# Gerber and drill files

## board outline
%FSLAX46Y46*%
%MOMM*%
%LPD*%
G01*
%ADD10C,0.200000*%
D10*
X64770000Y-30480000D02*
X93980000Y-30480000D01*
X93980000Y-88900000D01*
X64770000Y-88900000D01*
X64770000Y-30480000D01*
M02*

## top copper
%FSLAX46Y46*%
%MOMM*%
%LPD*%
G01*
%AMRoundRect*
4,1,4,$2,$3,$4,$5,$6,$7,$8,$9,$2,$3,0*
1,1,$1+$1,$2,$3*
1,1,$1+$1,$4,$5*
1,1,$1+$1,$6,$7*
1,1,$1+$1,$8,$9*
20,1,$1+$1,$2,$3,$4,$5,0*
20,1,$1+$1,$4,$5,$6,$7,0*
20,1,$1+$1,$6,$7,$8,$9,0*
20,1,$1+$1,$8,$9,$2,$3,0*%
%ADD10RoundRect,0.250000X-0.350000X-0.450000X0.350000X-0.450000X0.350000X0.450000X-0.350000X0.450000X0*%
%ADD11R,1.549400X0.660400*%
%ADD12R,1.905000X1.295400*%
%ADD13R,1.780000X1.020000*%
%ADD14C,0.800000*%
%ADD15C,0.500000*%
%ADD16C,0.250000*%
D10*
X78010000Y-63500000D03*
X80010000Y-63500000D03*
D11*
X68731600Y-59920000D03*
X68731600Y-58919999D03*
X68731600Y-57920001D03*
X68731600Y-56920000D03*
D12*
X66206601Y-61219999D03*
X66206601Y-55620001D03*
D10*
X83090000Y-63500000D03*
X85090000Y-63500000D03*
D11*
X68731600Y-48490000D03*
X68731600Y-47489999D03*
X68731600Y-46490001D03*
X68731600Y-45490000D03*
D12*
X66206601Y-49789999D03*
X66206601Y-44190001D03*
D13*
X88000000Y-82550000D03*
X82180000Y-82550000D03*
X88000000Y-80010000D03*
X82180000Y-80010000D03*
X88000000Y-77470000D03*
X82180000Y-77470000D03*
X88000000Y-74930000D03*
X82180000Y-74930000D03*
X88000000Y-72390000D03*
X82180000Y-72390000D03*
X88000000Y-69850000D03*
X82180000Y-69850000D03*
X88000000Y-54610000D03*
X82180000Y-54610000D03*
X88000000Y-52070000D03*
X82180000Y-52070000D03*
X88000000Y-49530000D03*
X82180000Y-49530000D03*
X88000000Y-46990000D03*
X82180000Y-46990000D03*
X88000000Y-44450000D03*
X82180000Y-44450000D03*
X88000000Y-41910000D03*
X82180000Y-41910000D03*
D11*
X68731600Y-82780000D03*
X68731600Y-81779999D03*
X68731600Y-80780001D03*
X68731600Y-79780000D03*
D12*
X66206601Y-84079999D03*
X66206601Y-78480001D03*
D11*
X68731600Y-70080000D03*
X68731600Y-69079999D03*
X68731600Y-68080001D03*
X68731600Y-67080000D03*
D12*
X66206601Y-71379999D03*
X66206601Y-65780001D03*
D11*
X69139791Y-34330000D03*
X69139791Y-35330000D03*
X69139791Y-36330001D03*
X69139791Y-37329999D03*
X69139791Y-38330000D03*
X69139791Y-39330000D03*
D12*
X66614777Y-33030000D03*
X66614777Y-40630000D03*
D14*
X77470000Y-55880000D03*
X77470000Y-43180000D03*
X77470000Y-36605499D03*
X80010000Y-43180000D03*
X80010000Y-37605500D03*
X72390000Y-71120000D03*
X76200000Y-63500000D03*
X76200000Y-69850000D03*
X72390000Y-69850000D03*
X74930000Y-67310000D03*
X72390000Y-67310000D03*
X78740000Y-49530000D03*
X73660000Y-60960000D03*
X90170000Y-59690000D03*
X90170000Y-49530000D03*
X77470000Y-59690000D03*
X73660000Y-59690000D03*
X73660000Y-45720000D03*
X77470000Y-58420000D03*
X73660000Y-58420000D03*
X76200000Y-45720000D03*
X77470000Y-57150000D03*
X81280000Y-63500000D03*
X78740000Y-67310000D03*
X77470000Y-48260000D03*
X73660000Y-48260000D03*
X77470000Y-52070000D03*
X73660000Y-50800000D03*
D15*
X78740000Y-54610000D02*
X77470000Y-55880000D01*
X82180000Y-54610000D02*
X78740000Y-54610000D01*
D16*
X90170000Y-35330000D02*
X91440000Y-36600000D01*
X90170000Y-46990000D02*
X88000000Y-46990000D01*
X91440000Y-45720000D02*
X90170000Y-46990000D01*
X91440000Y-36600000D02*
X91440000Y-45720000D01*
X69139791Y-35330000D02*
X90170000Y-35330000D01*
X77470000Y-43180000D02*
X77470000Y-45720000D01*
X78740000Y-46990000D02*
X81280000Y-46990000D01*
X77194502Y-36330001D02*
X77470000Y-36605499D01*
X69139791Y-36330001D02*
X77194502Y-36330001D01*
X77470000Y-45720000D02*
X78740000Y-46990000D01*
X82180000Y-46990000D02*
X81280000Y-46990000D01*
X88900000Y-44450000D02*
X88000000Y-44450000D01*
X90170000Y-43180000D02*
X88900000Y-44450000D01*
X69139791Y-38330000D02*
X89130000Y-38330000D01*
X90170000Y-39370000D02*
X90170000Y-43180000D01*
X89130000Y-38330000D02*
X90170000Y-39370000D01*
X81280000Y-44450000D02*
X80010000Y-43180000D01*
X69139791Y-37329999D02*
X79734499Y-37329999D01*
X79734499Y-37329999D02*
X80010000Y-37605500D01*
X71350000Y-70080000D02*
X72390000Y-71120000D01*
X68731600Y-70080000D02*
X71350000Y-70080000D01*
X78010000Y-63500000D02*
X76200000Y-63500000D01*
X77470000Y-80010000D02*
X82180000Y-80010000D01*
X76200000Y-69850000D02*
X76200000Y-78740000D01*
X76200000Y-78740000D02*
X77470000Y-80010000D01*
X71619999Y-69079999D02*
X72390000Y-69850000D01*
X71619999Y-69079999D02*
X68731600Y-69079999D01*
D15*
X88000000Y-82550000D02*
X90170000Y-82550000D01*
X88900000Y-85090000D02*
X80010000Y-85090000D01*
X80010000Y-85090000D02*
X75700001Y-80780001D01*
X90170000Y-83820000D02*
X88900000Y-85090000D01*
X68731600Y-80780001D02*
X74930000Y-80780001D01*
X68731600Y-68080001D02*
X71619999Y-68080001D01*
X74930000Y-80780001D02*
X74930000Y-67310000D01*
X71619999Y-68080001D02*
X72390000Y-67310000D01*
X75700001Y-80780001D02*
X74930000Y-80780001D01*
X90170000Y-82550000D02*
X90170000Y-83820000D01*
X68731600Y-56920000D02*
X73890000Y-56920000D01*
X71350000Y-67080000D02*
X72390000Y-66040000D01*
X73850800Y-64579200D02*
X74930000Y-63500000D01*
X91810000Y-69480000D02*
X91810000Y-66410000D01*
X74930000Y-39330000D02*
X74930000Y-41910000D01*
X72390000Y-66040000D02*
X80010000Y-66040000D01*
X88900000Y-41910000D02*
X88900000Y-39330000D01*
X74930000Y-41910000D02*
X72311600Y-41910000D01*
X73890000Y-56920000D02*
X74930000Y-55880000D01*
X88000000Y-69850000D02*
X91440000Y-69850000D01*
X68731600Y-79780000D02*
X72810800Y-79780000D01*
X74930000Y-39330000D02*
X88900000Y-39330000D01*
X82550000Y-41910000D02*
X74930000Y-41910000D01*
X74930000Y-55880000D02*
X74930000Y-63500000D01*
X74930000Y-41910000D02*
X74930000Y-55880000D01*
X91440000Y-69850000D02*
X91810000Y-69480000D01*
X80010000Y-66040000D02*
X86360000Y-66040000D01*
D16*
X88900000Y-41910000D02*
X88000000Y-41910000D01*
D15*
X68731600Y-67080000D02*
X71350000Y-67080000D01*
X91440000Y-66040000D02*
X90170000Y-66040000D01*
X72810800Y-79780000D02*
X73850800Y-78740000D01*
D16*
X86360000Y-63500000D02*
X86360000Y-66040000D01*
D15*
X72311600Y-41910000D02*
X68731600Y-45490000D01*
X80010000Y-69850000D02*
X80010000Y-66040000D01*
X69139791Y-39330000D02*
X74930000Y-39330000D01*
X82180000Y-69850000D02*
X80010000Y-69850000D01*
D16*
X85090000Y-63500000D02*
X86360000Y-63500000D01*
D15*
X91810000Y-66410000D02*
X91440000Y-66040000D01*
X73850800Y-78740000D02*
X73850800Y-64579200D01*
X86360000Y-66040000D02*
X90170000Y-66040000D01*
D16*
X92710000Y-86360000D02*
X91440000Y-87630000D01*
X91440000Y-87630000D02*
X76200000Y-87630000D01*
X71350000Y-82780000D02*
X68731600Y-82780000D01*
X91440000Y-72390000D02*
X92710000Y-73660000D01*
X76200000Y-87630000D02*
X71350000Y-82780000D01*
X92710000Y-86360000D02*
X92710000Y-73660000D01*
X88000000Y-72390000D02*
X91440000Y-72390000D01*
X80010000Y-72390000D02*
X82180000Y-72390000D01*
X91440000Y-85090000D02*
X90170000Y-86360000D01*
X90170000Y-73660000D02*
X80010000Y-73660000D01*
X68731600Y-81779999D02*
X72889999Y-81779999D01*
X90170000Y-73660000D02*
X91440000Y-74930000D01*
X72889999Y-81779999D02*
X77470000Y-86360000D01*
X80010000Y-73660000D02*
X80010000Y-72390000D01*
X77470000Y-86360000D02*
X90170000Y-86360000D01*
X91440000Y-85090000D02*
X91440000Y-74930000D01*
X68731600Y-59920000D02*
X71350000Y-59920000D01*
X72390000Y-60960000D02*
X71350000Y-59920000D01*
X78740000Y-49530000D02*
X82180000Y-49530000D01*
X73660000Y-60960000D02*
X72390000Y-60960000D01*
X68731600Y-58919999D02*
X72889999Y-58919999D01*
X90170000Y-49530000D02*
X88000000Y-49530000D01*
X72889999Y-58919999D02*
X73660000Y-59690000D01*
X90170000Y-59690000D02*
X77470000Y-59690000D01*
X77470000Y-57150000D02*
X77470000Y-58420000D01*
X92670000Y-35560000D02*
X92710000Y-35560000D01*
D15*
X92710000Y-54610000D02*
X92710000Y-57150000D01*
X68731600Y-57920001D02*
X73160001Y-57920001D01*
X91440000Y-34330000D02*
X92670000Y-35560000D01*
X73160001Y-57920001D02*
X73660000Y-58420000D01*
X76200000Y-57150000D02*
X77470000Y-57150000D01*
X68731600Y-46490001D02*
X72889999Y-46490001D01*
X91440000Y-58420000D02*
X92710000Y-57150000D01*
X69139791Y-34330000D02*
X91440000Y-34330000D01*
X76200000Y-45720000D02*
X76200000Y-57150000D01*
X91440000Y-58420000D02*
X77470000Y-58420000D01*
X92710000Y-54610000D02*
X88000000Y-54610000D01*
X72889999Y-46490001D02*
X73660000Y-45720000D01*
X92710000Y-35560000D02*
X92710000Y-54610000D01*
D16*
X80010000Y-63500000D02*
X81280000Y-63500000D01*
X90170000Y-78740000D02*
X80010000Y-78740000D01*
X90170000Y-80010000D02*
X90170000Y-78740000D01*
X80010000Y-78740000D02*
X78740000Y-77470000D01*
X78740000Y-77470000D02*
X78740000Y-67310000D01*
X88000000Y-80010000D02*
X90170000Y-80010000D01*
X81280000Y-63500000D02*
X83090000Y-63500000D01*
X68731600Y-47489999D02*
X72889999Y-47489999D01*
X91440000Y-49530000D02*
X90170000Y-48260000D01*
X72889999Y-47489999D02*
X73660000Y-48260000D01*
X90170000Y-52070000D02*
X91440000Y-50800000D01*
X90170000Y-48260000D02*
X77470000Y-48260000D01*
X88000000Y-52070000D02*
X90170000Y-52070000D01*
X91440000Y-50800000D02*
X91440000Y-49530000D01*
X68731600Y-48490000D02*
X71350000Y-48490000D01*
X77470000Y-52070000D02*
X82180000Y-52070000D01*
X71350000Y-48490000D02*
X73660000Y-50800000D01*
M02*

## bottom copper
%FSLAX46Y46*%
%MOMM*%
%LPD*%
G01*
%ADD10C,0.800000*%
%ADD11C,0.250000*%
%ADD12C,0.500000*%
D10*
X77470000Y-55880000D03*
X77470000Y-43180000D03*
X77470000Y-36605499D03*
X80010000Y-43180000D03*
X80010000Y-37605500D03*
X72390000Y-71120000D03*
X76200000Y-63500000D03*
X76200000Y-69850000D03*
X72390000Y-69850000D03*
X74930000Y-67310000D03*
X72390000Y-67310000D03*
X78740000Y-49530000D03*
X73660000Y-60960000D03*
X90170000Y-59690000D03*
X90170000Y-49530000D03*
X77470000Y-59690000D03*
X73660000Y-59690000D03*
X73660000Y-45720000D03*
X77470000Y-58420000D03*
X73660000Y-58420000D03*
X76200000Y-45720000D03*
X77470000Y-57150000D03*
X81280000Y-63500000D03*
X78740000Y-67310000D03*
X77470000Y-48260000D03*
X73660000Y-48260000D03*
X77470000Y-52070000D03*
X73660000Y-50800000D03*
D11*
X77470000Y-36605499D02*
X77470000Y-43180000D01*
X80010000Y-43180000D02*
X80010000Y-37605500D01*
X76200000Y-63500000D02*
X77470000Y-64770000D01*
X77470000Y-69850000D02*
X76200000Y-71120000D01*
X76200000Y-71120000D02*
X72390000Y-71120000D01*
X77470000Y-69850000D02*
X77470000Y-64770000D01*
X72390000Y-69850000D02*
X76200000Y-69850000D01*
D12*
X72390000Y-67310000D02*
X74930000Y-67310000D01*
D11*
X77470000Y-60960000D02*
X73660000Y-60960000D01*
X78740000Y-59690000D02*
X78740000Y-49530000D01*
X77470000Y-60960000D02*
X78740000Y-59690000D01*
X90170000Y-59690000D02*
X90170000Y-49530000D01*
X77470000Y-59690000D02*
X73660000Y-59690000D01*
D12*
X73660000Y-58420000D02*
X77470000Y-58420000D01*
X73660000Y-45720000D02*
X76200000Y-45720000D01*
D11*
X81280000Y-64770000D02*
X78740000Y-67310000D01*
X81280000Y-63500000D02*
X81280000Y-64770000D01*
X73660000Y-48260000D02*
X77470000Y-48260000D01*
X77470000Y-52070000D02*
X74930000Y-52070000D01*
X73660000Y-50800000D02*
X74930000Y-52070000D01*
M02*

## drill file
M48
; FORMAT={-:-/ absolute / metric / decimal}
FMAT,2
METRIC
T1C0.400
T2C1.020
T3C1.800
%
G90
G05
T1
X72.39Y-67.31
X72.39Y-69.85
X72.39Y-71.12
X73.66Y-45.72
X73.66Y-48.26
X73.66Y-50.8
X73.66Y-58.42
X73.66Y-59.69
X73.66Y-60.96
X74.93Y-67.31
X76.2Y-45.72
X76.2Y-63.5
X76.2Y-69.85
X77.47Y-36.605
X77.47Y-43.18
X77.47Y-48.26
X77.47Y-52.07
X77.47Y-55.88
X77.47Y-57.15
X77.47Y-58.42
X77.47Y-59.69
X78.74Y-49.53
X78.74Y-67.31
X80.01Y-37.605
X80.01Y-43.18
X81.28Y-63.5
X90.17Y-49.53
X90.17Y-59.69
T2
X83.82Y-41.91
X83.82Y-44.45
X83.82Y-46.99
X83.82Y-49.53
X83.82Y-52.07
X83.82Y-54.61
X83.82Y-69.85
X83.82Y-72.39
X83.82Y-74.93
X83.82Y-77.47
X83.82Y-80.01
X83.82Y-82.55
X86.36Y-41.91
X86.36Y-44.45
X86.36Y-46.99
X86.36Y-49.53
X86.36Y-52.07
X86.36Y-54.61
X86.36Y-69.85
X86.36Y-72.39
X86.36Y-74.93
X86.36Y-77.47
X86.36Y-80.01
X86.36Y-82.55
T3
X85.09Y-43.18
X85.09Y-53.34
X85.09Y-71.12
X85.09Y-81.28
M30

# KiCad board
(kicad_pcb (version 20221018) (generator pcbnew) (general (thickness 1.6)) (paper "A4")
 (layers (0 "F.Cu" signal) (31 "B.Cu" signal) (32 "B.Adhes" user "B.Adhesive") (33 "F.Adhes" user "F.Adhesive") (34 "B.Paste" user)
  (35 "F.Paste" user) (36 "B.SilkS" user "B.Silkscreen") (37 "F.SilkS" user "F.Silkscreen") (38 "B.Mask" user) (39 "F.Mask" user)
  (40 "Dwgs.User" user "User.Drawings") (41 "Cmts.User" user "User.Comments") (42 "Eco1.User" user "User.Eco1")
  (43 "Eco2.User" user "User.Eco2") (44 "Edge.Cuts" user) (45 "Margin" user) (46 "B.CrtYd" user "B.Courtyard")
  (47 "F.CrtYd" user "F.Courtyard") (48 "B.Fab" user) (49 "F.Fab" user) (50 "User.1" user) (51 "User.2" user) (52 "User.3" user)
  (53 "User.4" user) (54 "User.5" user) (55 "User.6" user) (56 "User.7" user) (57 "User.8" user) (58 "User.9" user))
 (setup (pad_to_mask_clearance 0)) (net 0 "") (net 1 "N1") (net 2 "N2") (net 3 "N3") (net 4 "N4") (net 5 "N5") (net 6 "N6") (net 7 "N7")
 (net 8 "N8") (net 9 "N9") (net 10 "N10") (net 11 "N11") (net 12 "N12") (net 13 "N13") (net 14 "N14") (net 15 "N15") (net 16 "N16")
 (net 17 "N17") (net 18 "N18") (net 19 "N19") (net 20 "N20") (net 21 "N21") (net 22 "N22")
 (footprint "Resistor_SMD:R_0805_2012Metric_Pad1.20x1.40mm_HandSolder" (layer "F.Cu") (at 79.01 63.5)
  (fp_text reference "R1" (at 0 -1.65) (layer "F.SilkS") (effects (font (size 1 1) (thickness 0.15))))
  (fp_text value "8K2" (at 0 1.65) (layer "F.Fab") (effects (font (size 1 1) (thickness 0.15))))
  (pad "1" smd roundrect (at -1 0) (size 1.2 1.4) (layers "F.Cu" "F.Paste" "F.Mask") (roundrect_rratio 0.2083333333) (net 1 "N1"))
  (pad "2" smd roundrect (at 1 0) (size 1.2 1.4) (layers "F.Cu" "F.Paste" "F.Mask") (roundrect_rratio 0.2083333333) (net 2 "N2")))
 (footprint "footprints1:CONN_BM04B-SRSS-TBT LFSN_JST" (layer "F.Cu") (at 67.31 58.42 90)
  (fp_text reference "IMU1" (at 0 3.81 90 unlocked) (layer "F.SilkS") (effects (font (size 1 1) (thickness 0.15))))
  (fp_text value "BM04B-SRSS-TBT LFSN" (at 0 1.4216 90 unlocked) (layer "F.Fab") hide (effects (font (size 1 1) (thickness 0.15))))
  (pad "1" smd rect (at -1.5 1.4216 90) (size 0.6604 1.5494) (layers "F.Cu" "F.Paste" "F.Mask") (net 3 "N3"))
  (pad "2" smd rect (at -0.499999 1.4216 90) (size 0.6604 1.5494) (layers "F.Cu" "F.Paste" "F.Mask") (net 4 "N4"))
  (pad "3" smd rect (at 0.499999 1.4216 90) (size 0.6604 1.5494) (layers "F.Cu" "F.Paste" "F.Mask") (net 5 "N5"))
  (pad "4" smd rect (at 1.5 1.4216 90) (size 0.6604 1.5494) (layers "F.Cu" "F.Paste" "F.Mask") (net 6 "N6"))
  (pad "5" smd rect (at -2.799999 -1.103399 180) (size 1.905 1.2954) (layers "F.Cu" "F.Paste" "F.Mask"))
  (pad "6" smd rect (at 2.799999 -1.103399 180) (size 1.905 1.2954) (layers "F.Cu" "F.Paste" "F.Mask")))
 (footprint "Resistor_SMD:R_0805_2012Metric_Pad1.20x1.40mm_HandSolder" (layer "F.Cu") (at 84.09 63.5)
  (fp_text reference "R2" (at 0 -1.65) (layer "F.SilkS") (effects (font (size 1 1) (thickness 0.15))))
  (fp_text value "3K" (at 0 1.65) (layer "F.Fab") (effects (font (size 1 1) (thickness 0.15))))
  (pad "1" smd roundrect (at -1 0) (size 1.2 1.4) (layers "F.Cu" "F.Paste" "F.Mask") (roundrect_rratio 0.2083333333) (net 2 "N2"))
  (pad "2" smd roundrect (at 1 0) (size 1.2 1.4) (layers "F.Cu" "F.Paste" "F.Mask") (roundrect_rratio 0.2083333333) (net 6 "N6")))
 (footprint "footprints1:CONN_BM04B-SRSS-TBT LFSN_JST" (layer "F.Cu") (at 67.31 46.99 90)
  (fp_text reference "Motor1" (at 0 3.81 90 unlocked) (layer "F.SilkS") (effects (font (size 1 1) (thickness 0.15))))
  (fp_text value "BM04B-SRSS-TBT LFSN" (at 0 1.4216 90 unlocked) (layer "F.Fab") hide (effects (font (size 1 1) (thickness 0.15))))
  (pad "1" smd rect (at -1.5 1.4216 90) (size 0.6604 1.5494) (layers "F.Cu" "F.Paste" "F.Mask") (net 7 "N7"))
  (pad "2" smd rect (at -0.499999 1.4216 90) (size 0.6604 1.5494) (layers "F.Cu" "F.Paste" "F.Mask") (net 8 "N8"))
  (pad "3" smd rect (at 0.499999 1.4216 90) (size 0.6604 1.5494) (layers "F.Cu" "F.Paste" "F.Mask") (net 5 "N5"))
  (pad "4" smd rect (at 1.5 1.4216 90) (size 0.6604 1.5494) (layers "F.Cu" "F.Paste" "F.Mask") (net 6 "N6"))
  (pad "5" smd rect (at -2.799999 -1.103399 180) (size 1.905 1.2954) (layers "F.Cu" "F.Paste" "F.Mask"))
  (pad "6" smd rect (at 2.799999 -1.103399 180) (size 1.905 1.2954) (layers "F.Cu" "F.Paste" "F.Mask")))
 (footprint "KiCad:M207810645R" (layer "F.Cu") (at 85.09 76.2 90)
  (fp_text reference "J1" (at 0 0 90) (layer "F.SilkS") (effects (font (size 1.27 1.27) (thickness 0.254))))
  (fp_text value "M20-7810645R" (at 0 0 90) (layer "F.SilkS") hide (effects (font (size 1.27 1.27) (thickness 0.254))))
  (pad "" np_thru_hole circle (at -6.35 -1.27 90) (size 1.02 1.02) (drill 1.02) (layers "*.Cu" "*.Mask"))
  (pad "" np_thru_hole circle (at -6.35 1.27 90) (size 1.02 1.02) (drill 1.02) (layers "*.Cu" "*.Mask"))
  (pad "" np_thru_hole circle (at -5.08 0 90) (size 1.8 1.8) (drill 1.8) (layers "*.Cu" "*.Mask"))
  (pad "" np_thru_hole circle (at -3.81 -1.27 90) (size 1.02 1.02) (drill 1.02) (layers "*.Cu" "*.Mask"))
  (pad "" np_thru_hole circle (at -3.81 1.27 90) (size 1.02 1.02) (drill 1.02) (layers "*.Cu" "*.Mask"))
  (pad "" np_thru_hole circle (at -1.27 -1.27 90) (size 1.02 1.02) (drill 1.02) (layers "*.Cu" "*.Mask"))
  (pad "" np_thru_hole circle (at -1.27 1.27 90) (size 1.02 1.02) (drill 1.02) (layers "*.Cu" "*.Mask"))
  (pad "" np_thru_hole circle (at 1.27 -1.27 90) (size 1.02 1.02) (drill 1.02) (layers "*.Cu" "*.Mask"))
  (pad "" np_thru_hole circle (at 1.27 1.27 90) (size 1.02 1.02) (drill 1.02) (layers "*.Cu" "*.Mask"))
  (pad "" np_thru_hole circle (at 3.81 -1.27 90) (size 1.02 1.02) (drill 1.02) (layers "*.Cu" "*.Mask"))
  (pad "" np_thru_hole circle (at 3.81 1.27 90) (size 1.02 1.02) (drill 1.02) (layers "*.Cu" "*.Mask"))
  (pad "" np_thru_hole circle (at 5.08 0 90) (size 1.8 1.8) (drill 1.8) (layers "*.Cu" "*.Mask"))
  (pad "" np_thru_hole circle (at 6.35 -1.27 90) (size 1.02 1.02) (drill 1.02) (layers "*.Cu" "*.Mask"))
  (pad "" np_thru_hole circle (at 6.35 1.27 90) (size 1.02 1.02) (drill 1.02) (layers "*.Cu" "*.Mask"))
  (pad "1" smd rect (at -6.35 2.91 90) (size 1.02 1.78) (layers "F.Cu" "F.Paste" "F.Mask") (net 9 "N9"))
  (pad "2" smd rect (at -6.35 -2.91 90) (size 1.02 1.78) (layers "F.Cu" "F.Paste" "F.Mask") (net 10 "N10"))
  (pad "3" smd rect (at -3.81 2.91 90) (size 1.02 1.78) (layers "F.Cu" "F.Paste" "F.Mask") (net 2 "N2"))
  (pad "4" smd rect (at -3.81 -2.91 90) (size 1.02 1.78) (layers "F.Cu" "F.Paste" "F.Mask") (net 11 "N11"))
  (pad "5" smd rect (at -1.27 2.91 90) (size 1.02 1.78) (layers "F.Cu" "F.Paste" "F.Mask") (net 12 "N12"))
  (pad "6" smd rect (at -1.27 -2.91 90) (size 1.02 1.78) (layers "F.Cu" "F.Paste" "F.Mask") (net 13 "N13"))
  (pad "7" smd rect (at 1.27 2.91 90) (size 1.02 1.78) (layers "F.Cu" "F.Paste" "F.Mask") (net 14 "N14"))
  (pad "8" smd rect (at 1.27 -2.91 90) (size 1.02 1.78) (layers "F.Cu" "F.Paste" "F.Mask") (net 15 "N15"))
  (pad "9" smd rect (at 3.81 2.91 90) (size 1.02 1.78) (layers "F.Cu" "F.Paste" "F.Mask") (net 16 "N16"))
  (pad "10" smd rect (at 3.81 -2.91 90) (size 1.02 1.78) (layers "F.Cu" "F.Paste" "F.Mask") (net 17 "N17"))
  (pad "11" smd rect (at 6.35 2.91 90) (size 1.02 1.78) (layers "F.Cu" "F.Paste" "F.Mask") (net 6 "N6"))
  (pad "12" smd rect (at 6.35 -2.91 90) (size 1.02 1.78) (layers "F.Cu" "F.Paste" "F.Mask") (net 6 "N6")))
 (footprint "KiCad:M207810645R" (layer "F.Cu") (at 85.09 48.26 90)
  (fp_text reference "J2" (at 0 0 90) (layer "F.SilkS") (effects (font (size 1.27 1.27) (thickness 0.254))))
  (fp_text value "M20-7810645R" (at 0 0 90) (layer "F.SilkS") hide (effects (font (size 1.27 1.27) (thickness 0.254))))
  (pad "" np_thru_hole circle (at -6.35 -1.27 90) (size 1.02 1.02) (drill 1.02) (layers "*.Cu" "*.Mask"))
  (pad "" np_thru_hole circle (at -6.35 1.27 90) (size 1.02 1.02) (drill 1.02) (layers "*.Cu" "*.Mask"))
  (pad "" np_thru_hole circle (at -5.08 0 90) (size 1.8 1.8) (drill 1.8) (layers "*.Cu" "*.Mask"))
  (pad "" np_thru_hole circle (at -3.81 -1.27 90) (size 1.02 1.02) (drill 1.02) (layers "*.Cu" "*.Mask"))
  (pad "" np_thru_hole circle (at -3.81 1.27 90) (size 1.02 1.02) (drill 1.02) (layers "*.Cu" "*.Mask"))
  (pad "" np_thru_hole circle (at -1.27 -1.27 90) (size 1.02 1.02) (drill 1.02) (layers "*.Cu" "*.Mask"))
  (pad "" np_thru_hole circle (at -1.27 1.27 90) (size 1.02 1.02) (drill 1.02) (layers "*.Cu" "*.Mask"))
  (pad "" np_thru_hole circle (at 1.27 -1.27 90) (size 1.02 1.02) (drill 1.02) (layers "*.Cu" "*.Mask"))
  (pad "" np_thru_hole circle (at 1.27 1.27 90) (size 1.02 1.02) (drill 1.02) (layers "*.Cu" "*.Mask"))
  (pad "" np_thru_hole circle (at 3.81 -1.27 90) (size 1.02 1.02) (drill 1.02) (layers "*.Cu" "*.Mask"))
  (pad "" np_thru_hole circle (at 3.81 1.27 90) (size 1.02 1.02) (drill 1.02) (layers "*.Cu" "*.Mask"))
  (pad "" np_thru_hole circle (at 5.08 0 90) (size 1.8 1.8) (drill 1.8) (layers "*.Cu" "*.Mask"))
  (pad "" np_thru_hole circle (at 6.35 -1.27 90) (size 1.02 1.02) (drill 1.02) (layers "*.Cu" "*.Mask"))
  (pad "" np_thru_hole circle (at 6.35 1.27 90) (size 1.02 1.02) (drill 1.02) (layers "*.Cu" "*.Mask"))
  (pad "1" smd rect (at -6.35 2.91 90) (size 1.02 1.78) (layers "F.Cu" "F.Paste" "F.Mask") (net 5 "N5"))
  (pad "2" smd rect (at -6.35 -2.91 90) (size 1.02 1.78) (layers "F.Cu" "F.Paste" "F.Mask") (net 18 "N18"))
  (pad "3" smd rect (at -3.81 2.91 90) (size 1.02 1.78) (layers "F.Cu" "F.Paste" "F.Mask") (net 8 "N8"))
  (pad "4" smd rect (at -3.81 -2.91 90) (size 1.02 1.78) (layers "F.Cu" "F.Paste" "F.Mask") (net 7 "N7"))
  (pad "5" smd rect (at -1.27 2.91 90) (size 1.02 1.78) (layers "F.Cu" "F.Paste" "F.Mask") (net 4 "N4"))
  (pad "6" smd rect (at -1.27 -2.91 90) (size 1.02 1.78) (layers "F.Cu" "F.Paste" "F.Mask") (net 3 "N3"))
  (pad "7" smd rect (at 1.27 2.91 90) (size 1.02 1.78) (layers "F.Cu" "F.Paste" "F.Mask") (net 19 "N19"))
  (pad "8" smd rect (at 1.27 -2.91 90) (size 1.02 1.78) (layers "F.Cu" "F.Paste" "F.Mask") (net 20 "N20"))
  (pad "9" smd rect (at 3.81 2.91 90) (size 1.02 1.78) (layers "F.Cu" "F.Paste" "F.Mask") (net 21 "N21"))
  (pad "10" smd rect (at 3.81 -2.91 90) (size 1.02 1.78) (layers "F.Cu" "F.Paste" "F.Mask") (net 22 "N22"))
  (pad "11" smd rect (at 6.35 2.91 90) (size 1.02 1.78) (layers "F.Cu" "F.Paste" "F.Mask") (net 6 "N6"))
  (pad "12" smd rect (at 6.35 -2.91 90) (size 1.02 1.78) (layers "F.Cu" "F.Paste" "F.Mask") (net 6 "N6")))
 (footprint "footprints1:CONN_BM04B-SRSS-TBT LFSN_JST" (layer "F.Cu") (at 67.31 81.28 90)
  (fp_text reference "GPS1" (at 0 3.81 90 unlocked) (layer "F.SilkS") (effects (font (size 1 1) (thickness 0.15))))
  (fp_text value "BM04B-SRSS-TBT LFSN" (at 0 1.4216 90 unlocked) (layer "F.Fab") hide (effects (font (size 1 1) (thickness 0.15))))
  (pad "1" smd rect (at -1.5 1.4216 90) (size 0.6604 1.5494) (layers "F.Cu" "F.Paste" "F.Mask") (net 16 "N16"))
  (pad "2" smd rect (at -0.499999 1.4216 90) (size 0.6604 1.5494) (layers "F.Cu" "F.Paste" "F.Mask") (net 17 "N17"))
  (pad "3" smd rect (at 0.499999 1.4216 90) (size 0.6604 1.5494) (layers "F.Cu" "F.Paste" "F.Mask") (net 9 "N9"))
  (pad "4" smd rect (at 1.5 1.4216 90) (size 0.6604 1.5494) (layers "F.Cu" "F.Paste" "F.Mask") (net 6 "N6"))
  (pad "5" smd rect (at -2.799999 -1.103399 180) (size 1.905 1.2954) (layers "F.Cu" "F.Paste" "F.Mask"))
  (pad "6" smd rect (at 2.799999 -1.103399 180) (size 1.905 1.2954) (layers "F.Cu" "F.Paste" "F.Mask")))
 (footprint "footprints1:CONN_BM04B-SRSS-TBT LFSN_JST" (layer "F.Cu") (at 67.31 68.58 90)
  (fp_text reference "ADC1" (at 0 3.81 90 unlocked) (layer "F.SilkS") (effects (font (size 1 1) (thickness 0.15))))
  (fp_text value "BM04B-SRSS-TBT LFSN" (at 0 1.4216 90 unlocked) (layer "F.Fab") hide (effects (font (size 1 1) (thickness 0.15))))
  (pad "1" smd rect (at -1.5 1.4216 90) (size 0.6604 1.5494) (layers "F.Cu" "F.Paste" "F.Mask") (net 1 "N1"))
  (pad "2" smd rect (at -0.499999 1.4216 90) (size 0.6604 1.5494) (layers "F.Cu" "F.Paste" "F.Mask") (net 11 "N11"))
  (pad "3" smd rect (at 0.499999 1.4216 90) (size 0.6604 1.5494) (layers "F.Cu" "F.Paste" "F.Mask") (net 9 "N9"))
  (pad "4" smd rect (at 1.5 1.4216 90) (size 0.6604 1.5494) (layers "F.Cu" "F.Paste" "F.Mask") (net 6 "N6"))
  (pad "5" smd rect (at -2.799999 -1.103399 180) (size 1.905 1.2954) (layers "F.Cu" "F.Paste" "F.Mask"))
  (pad "6" smd rect (at 2.799999 -1.103399 180) (size 1.905 1.2954) (layers "F.Cu" "F.Paste" "F.Mask")))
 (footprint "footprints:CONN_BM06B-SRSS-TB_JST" (layer "F.Cu") (at 67.31 36.83 -90)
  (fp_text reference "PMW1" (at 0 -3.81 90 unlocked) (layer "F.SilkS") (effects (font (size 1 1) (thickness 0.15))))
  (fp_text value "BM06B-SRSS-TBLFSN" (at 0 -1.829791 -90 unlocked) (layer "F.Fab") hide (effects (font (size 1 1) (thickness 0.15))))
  (pad "1" smd rect (at -2.5 -1.829791 270) (size 0.6604 1.5494) (layers "F.Cu" "F.Paste" "F.Mask") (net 5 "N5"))
  (pad "2" smd rect (at -1.5 -1.829791 270) (size 0.6604 1.5494) (layers "F.Cu" "F.Paste" "F.Mask") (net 19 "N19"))
  (pad "3" smd rect (at -0.499999 -1.829791 270) (size 0.6604 1.5494) (layers "F.Cu" "F.Paste" "F.Mask") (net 20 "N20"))
  (pad "4" smd rect (at 0.499999 -1.829791 270) (size 0.6604 1.5494) (layers "F.Cu" "F.Paste" "F.Mask") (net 22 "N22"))
  (pad "5" smd rect (at 1.5 -1.829791 270) (size 0.6604 1.5494) (layers "F.Cu" "F.Paste" "F.Mask") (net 21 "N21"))
  (pad "6" smd rect (at 2.5 -1.829791 270) (size 0.6604 1.5494) (layers "F.Cu" "F.Paste" "F.Mask") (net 6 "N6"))
  (pad "7" smd rect (at -3.8 0.695223) (size 1.905 1.2954) (layers "F.Cu" "F.Paste" "F.Mask"))
  (pad "8" smd rect (at 3.8 0.695223) (size 1.905 1.2954) (layers "F.Cu" "F.Paste" "F.Mask")))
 (gr_rect (start 64.77 30.48) (end 93.98 88.9) (stroke (width 0.2) (type default)) (fill none) (layer "Edge.Cuts"))
 (segment (start 78.74 54.61) (end 77.47 55.88) (width 0.5) (layer "F.Cu") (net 18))
 (segment (start 82.18 54.61) (end 78.74 54.61) (width 0.5) (layer "F.Cu") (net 18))
 (via (at 77.47 55.88) (size 0.8) (drill 0.4) (layers "F.Cu" "B.Cu") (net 18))
 (segment (start 90.17 35.33) (end 91.44 36.6) (width 0.25) (layer "F.Cu") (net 19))
 (segment (start 90.17 46.99) (end 88 46.99) (width 0.25) (layer "F.Cu") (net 19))
 (segment (start 91.44 45.72) (end 90.17 46.99) (width 0.25) (layer "F.Cu") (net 19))
 (segment (start 91.44 36.6) (end 91.44 45.72) (width 0.25) (layer "F.Cu") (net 19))
 (segment (start 69.139791 35.33) (end 90.17 35.33) (width 0.25) (layer "F.Cu") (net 19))
 (segment (start 77.47 43.18) (end 77.47 45.72) (width 0.25) (layer "F.Cu") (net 20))
 (segment (start 78.74 46.99) (end 81.28 46.99) (width 0.25) (layer "F.Cu") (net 20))
 (segment (start 77.194502 36.330001) (end 77.47 36.605499) (width 0.25) (layer "F.Cu") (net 20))
 (segment (start 69.139791 36.330001) (end 77.194502 36.330001) (width 0.25) (layer "F.Cu") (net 20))
 (segment (start 77.47 45.72) (end 78.74 46.99) (width 0.25) (layer "F.Cu") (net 20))
 (segment (start 82.18 46.99) (end 81.28 46.99) (width 0.25) (layer "F.Cu") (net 20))
 (via (at 77.47 43.18) (size 0.8) (drill 0.4) (layers "F.Cu" "B.Cu") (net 20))
 (via (at 77.47 36.605499) (size 0.8) (drill 0.4) (layers "F.Cu" "B.Cu") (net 20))
 (segment (start 77.47 36.605499) (end 77.47 43.18) (width 0.25) (layer "B.Cu") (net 20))
 (segment (start 88.9 44.45) (end 88 44.45) (width 0.25) (layer "F.Cu") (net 21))
 (segment (start 90.17 43.18) (end 88.9 44.45) (width 0.25) (layer "F.Cu") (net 21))
 (segment (start 69.139791 38.33) (end 89.13 38.33) (width 0.25) (layer "F.Cu") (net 21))
 (segment (start 90.17 39.37) (end 90.17 43.18) (width 0.25) (layer "F.Cu") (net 21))
 (segment (start 89.13 38.33) (end 90.17 39.37) (width 0.25) (layer "F.Cu") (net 21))
 (segment (start 81.28 44.45) (end 80.01 43.18) (width 0.25) (layer "F.Cu") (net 22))
 (segment (start 69.139791 37.329999) (end 79.734499 37.329999) (width 0.25) (layer "F.Cu") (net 22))
 (segment (start 79.734499 37.329999) (end 80.01 37.6055) (width 0.25) (layer "F.Cu") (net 22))
 (via (at 80.01 43.18) (size 0.8) (drill 0.4) (layers "F.Cu" "B.Cu") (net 22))
 (via (at 80.01 37.6055) (size 0.8) (drill 0.4) (layers "F.Cu" "B.Cu") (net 22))
 (segment (start 80.01 43.18) (end 80.01 37.6055) (width 0.25) (layer "B.Cu") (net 22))
 (segment (start 71.35 70.08) (end 72.39 71.12) (width 0.25) (layer "F.Cu") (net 1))
 (segment (start 68.7316 70.08) (end 71.35 70.08) (width 0.25) (layer "F.Cu") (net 1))
 (segment (start 78.01 63.5) (end 76.2 63.5) (width 0.25) (layer "F.Cu") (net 1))
 (via (at 72.39 71.12) (size 0.8) (drill 0.4) (layers "F.Cu" "B.Cu") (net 1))
 (via (at 76.2 63.5) (size 0.8) (drill 0.4) (layers "F.Cu" "B.Cu") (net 1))
 (segment (start 76.2 63.5) (end 77.47 64.77) (width 0.25) (layer "B.Cu") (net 1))
 (segment (start 77.47 69.85) (end 76.2 71.12) (width 0.25) (layer "B.Cu") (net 1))
 (segment (start 76.2 71.12) (end 72.39 71.12) (width 0.25) (layer "B.Cu") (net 1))
 (segment (start 77.47 69.85) (end 77.47 64.77) (width 0.25) (layer "B.Cu") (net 1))
 (segment (start 77.47 80.01) (end 82.18 80.01) (width 0.25) (layer "F.Cu") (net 11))
 (segment (start 76.2 69.85) (end 76.2 78.74) (width 0.25) (layer "F.Cu") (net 11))
 (segment (start 76.2 78.74) (end 77.47 80.01) (width 0.25) (layer "F.Cu") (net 11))
 (segment (start 71.619999 69.079999) (end 72.39 69.85) (width 0.25) (layer "F.Cu") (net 11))
 (segment (start 71.619999 69.079999) (end 68.7316 69.079999) (width 0.25) (layer "F.Cu") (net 11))
 (via (at 76.2 69.85) (size 0.8) (drill 0.4) (layers "F.Cu" "B.Cu") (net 11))
 (via (at 72.39 69.85) (size 0.8) (drill 0.4) (layers "F.Cu" "B.Cu") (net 11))
 (segment (start 72.39 69.85) (end 76.2 69.85) (width 0.25) (layer "B.Cu") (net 11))
 (segment (start 88 82.55) (end 90.17 82.55) (width 0.5) (layer "F.Cu") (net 9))
 (segment (start 88.9 85.09) (end 80.01 85.09) (width 0.5) (layer "F.Cu") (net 9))
 (segment (start 80.01 85.09) (end 75.700001 80.780001) (width 0.5) (layer "F.Cu") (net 9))
 (segment (start 90.17 83.82) (end 88.9 85.09) (width 0.5) (layer "F.Cu") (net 9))
 (segment (start 68.7316 80.780001) (end 74.93 80.780001) (width 0.5) (layer "F.Cu") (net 9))
 (segment (start 68.7316 68.080001) (end 71.619999 68.080001) (width 0.5) (layer "F.Cu") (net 9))
 (segment (start 74.93 80.780001) (end 74.93 67.31) (width 0.5) (layer "F.Cu") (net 9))
 (segment (start 71.619999 68.080001) (end 72.39 67.31) (width 0.5) (layer "F.Cu") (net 9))
 (segment (start 75.700001 80.780001) (end 74.93 80.780001) (width 0.5) (layer "F.Cu") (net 9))
 (segment (start 90.17 82.55) (end 90.17 83.82) (width 0.5) (layer "F.Cu") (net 9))
 (via (at 74.93 67.31) (size 0.8) (drill 0.4) (layers "F.Cu" "B.Cu") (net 9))
 (via (at 72.39 67.31) (size 0.8) (drill 0.4) (layers "F.Cu" "B.Cu") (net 9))
 (segment (start 72.39 67.31) (end 74.93 67.31) (width 0.5) (layer "B.Cu") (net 9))
 (segment (start 68.7316 56.92) (end 73.89 56.92) (width 0.5) (layer "F.Cu") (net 6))
 (segment (start 71.35 67.08) (end 72.39 66.04) (width 0.5) (layer "F.Cu") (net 6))
 (segment (start 73.8508 64.5792) (end 74.93 63.5) (width 0.5) (layer "F.Cu") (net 6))
 (segment (start 91.81 69.48) (end 91.81 66.41) (width 0.5) (layer "F.Cu") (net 6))
 (segment (start 74.93 39.33) (end 74.93 41.91) (width 0.5) (layer "F.Cu") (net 6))
 (segment (start 72.39 66.04) (end 80.01 66.04) (width 0.5) (layer "F.Cu") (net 6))
 (segment (start 88.9 41.91) (end 88.9 39.33) (width 0.5) (layer "F.Cu") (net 6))
 (segment (start 74.93 41.91) (end 72.3116 41.91) (width 0.5) (layer "F.Cu") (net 6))
 (segment (start 73.89 56.92) (end 74.93 55.88) (width 0.5) (layer "F.Cu") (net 6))
 (segment (start 88 69.85) (end 91.44 69.85) (width 0.5) (layer "F.Cu") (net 6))
 (segment (start 68.7316 79.78) (end 72.8108 79.78) (width 0.5) (layer "F.Cu") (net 6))
 (segment (start 74.93 39.33) (end 88.9 39.33) (width 0.5) (layer "F.Cu") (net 6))
 (segment (start 82.55 41.91) (end 74.93 41.91) (width 0.5) (layer "F.Cu") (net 6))
 (segment (start 74.93 55.88) (end 74.93 63.5) (width 0.5) (layer "F.Cu") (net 6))
 (segment (start 74.93 41.91) (end 74.93 55.88) (width 0.5) (layer "F.Cu") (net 6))
 (segment (start 91.44 69.85) (end 91.81 69.48) (width 0.5) (layer "F.Cu") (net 6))
 (segment (start 80.01 66.04) (end 86.36 66.04) (width 0.5) (layer "F.Cu") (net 6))
 (segment (start 88.9 41.91) (end 88 41.91) (width 0.25) (layer "F.Cu") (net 6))
 (segment (start 68.7316 67.08) (end 71.35 67.08) (width 0.5) (layer "F.Cu") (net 6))
 (segment (start 91.44 66.04) (end 90.17 66.04) (width 0.5) (layer "F.Cu") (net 6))
 (segment (start 72.8108 79.78) (end 73.8508 78.74) (width 0.5) (layer "F.Cu") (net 6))
 (segment (start 86.36 63.5) (end 86.36 66.04) (width 0.25) (layer "F.Cu") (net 6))
 (segment (start 72.3116 41.91) (end 68.7316 45.49) (width 0.5) (layer "F.Cu") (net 6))
 (segment (start 80.01 69.85) (end 80.01 66.04) (width 0.5) (layer "F.Cu") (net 6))
 (segment (start 69.139791 39.33) (end 74.93 39.33) (width 0.5) (layer "F.Cu") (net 6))
 (segment (start 82.18 69.85) (end 80.01 69.85) (width 0.5) (layer "F.Cu") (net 6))
 (segment (start 85.09 63.5) (end 86.36 63.5) (width 0.25) (layer "F.Cu") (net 6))
 (segment (start 91.81 66.41) (end 91.44 66.04) (width 0.5) (layer "F.Cu") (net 6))
 (segment (start 73.8508 78.74) (end 73.8508 64.5792) (width 0.5) (layer "F.Cu") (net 6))
 (segment (start 86.36 66.04) (end 90.17 66.04) (width 0.5) (layer "F.Cu") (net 6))
 (segment (start 92.71 86.36) (end 91.44 87.63) (width 0.25) (layer "F.Cu") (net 16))
 (segment (start 91.44 87.63) (end 76.2 87.63) (width 0.25) (layer "F.Cu") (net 16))
 (segment (start 71.35 82.78) (end 68.7316 82.78) (width 0.25) (layer "F.Cu") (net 16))
 (segment (start 91.44 72.39) (end 92.71 73.66) (width 0.25) (layer "F.Cu") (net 16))
 (segment (start 76.2 87.63) (end 71.35 82.78) (width 0.25) (layer "F.Cu") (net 16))
 (segment (start 92.71 86.36) (end 92.71 73.66) (width 0.25) (layer "F.Cu") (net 16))
 (segment (start 88 72.39) (end 91.44 72.39) (width 0.25) (layer "F.Cu") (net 16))
 (segment (start 80.01 72.39) (end 82.18 72.39) (width 0.25) (layer "F.Cu") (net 17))
 (segment (start 91.44 85.09) (end 90.17 86.36) (width 0.25) (layer "F.Cu") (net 17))
 (segment (start 90.17 73.66) (end 80.01 73.66) (width 0.25) (layer "F.Cu") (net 17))
 (segment (start 68.7316 81.779999) (end 72.889999 81.779999) (width 0.25) (layer "F.Cu") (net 17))
 (segment (start 90.17 73.66) (end 91.44 74.93) (width 0.25) (layer "F.Cu") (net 17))
 (segment (start 72.889999 81.779999) (end 77.47 86.36) (width 0.25) (layer "F.Cu") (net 17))
 (segment (start 80.01 73.66) (end 80.01 72.39) (width 0.25) (layer "F.Cu") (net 17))
 (segment (start 77.47 86.36) (end 90.17 86.36) (width 0.25) (layer "F.Cu") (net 17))
 (segment (start 91.44 85.09) (end 91.44 74.93) (width 0.25) (layer "F.Cu") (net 17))
 (segment (start 68.7316 59.92) (end 71.35 59.92) (width 0.25) (layer "F.Cu") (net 3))
 (segment (start 72.39 60.96) (end 71.35 59.92) (width 0.25) (layer "F.Cu") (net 3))
 (segment (start 78.74 49.53) (end 82.18 49.53) (width 0.25) (layer "F.Cu") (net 3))
 (segment (start 73.66 60.96) (end 72.39 60.96) (width 0.25) (layer "F.Cu") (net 3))
 (via (at 78.74 49.53) (size 0.8) (drill 0.4) (layers "F.Cu" "B.Cu") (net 3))
 (via (at 73.66 60.96) (size 0.8) (drill 0.4) (layers "F.Cu" "B.Cu") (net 3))
 (segment (start 77.47 60.96) (end 73.66 60.96) (width 0.25) (layer "B.Cu") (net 3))
 (segment (start 78.74 59.69) (end 78.74 49.53) (width 0.25) (layer "B.Cu") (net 3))
 (segment (start 77.47 60.96) (end 78.74 59.69) (width 0.25) (layer "B.Cu") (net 3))
 (segment (start 68.7316 58.919999) (end 72.889999 58.919999) (width 0.25) (layer "F.Cu") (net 4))
 (segment (start 90.17 49.53) (end 88 49.53) (width 0.25) (layer "F.Cu") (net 4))
 (segment (start 72.889999 58.919999) (end 73.66 59.69) (width 0.25) (layer "F.Cu") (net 4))
 (segment (start 90.17 59.69) (end 77.47 59.69) (width 0.25) (layer "F.Cu") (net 4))
 (via (at 90.17 59.69) (size 0.8) (drill 0.4) (layers "F.Cu" "B.Cu") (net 4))
 (via (at 90.17 49.53) (size 0.8) (drill 0.4) (layers "F.Cu" "B.Cu") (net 4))
 (via (at 77.47 59.69) (size 0.8) (drill 0.4) (layers "F.Cu" "B.Cu") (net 4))
 (via (at 73.66 59.69) (size 0.8) (drill 0.4) (layers "F.Cu" "B.Cu") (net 4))
 (segment (start 90.17 59.69) (end 90.17 49.53) (width 0.25) (layer "B.Cu") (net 4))
 (segment (start 77.47 59.69) (end 73.66 59.69) (width 0.25) (layer "B.Cu") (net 4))
 (segment (start 77.47 57.15) (end 77.47 58.42) (width 0.25) (layer "F.Cu") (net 5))
 (segment (start 92.67 35.56) (end 92.71 35.56) (width 0.25) (layer "F.Cu") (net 5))
 (segment (start 92.71 54.61) (end 92.71 57.15) (width 0.5) (layer "F.Cu") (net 5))
 (segment (start 68.7316 57.920001) (end 73.160001 57.920001) (width 0.5) (layer "F.Cu") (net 5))
 (segment (start 91.44 34.33) (end 92.67 35.56) (width 0.5) (layer "F.Cu") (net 5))
 (segment (start 73.160001 57.920001) (end 73.66 58.42) (width 0.5) (layer "F.Cu") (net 5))
 (segment (start 76.2 57.15) (end 77.47 57.15) (width 0.5) (layer "F.Cu") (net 5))
 (segment (start 68.7316 46.490001) (end 72.889999 46.490001) (width 0.5) (layer "F.Cu") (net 5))
 (segment (start 91.44 58.42) (end 92.71 57.15) (width 0.5) (layer "F.Cu") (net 5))
 (segment (start 69.139791 34.33) (end 91.44 34.33) (width 0.5) (layer "F.Cu") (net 5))
 (segment (start 76.2 45.72) (end 76.2 57.15) (width 0.5) (layer "F.Cu") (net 5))
 (segment (start 91.44 58.42) (end 77.47 58.42) (width 0.5) (layer "F.Cu") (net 5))
 (segment (start 92.71 54.61) (end 88 54.61) (width 0.5) (layer "F.Cu") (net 5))
 (segment (start 72.889999 46.490001) (end 73.66 45.72) (width 0.5) (layer "F.Cu") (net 5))
 (segment (start 92.71 35.56) (end 92.71 54.61) (width 0.5) (layer "F.Cu") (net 5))
 (via (at 73.66 45.72) (size 0.8) (drill 0.4) (layers "F.Cu" "B.Cu") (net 5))
 (via (at 77.47 58.42) (size 0.8) (drill 0.4) (layers "F.Cu" "B.Cu") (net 5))
 (via (at 73.66 58.42) (size 0.8) (drill 0.4) (layers "F.Cu" "B.Cu") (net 5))
 (via (at 76.2 45.72) (size 0.8) (drill 0.4) (layers "F.Cu" "B.Cu") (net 5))
 (via (at 77.47 57.15) (size 0.8) (drill 0.4) (layers "F.Cu" "B.Cu") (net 5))
 (segment (start 73.66 58.42) (end 77.47 58.42) (width 0.5) (layer "B.Cu") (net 5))
 (segment (start 73.66 45.72) (end 76.2 45.72) (width 0.5) (layer "B.Cu") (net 5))
 (segment (start 80.01 63.5) (end 81.28 63.5) (width 0.25) (layer "F.Cu") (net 2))
 (segment (start 90.17 78.74) (end 80.01 78.74) (width 0.25) (layer "F.Cu") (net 2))
 (segment (start 90.17 80.01) (end 90.17 78.74) (width 0.25) (layer "F.Cu") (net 2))
 (segment (start 80.01 78.74) (end 78.74 77.47) (width 0.25) (layer "F.Cu") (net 2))
 (segment (start 78.74 77.47) (end 78.74 67.31) (width 0.25) (layer "F.Cu") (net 2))
 (segment (start 88 80.01) (end 90.17 80.01) (width 0.25) (layer "F.Cu") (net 2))
 (segment (start 81.28 63.5) (end 83.09 63.5) (width 0.25) (layer "F.Cu") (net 2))
 (via (at 81.28 63.5) (size 0.8) (drill 0.4) (layers "F.Cu" "B.Cu") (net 2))
 (via (at 78.74 67.31) (size 0.8) (drill 0.4) (layers "F.Cu" "B.Cu") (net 2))
 (segment (start 81.28 64.77) (end 78.74 67.31) (width 0.25) (layer "B.Cu") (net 2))
 (segment (start 81.28 63.5) (end 81.28 64.77) (width 0.25) (layer "B.Cu") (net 2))
 (segment (start 68.7316 47.489999) (end 72.889999 47.489999) (width 0.25) (layer "F.Cu") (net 8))
 (segment (start 91.44 49.53) (end 90.17 48.26) (width 0.25) (layer "F.Cu") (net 8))
 (segment (start 72.889999 47.489999) (end 73.66 48.26) (width 0.25) (layer "F.Cu") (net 8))
 (segment (start 90.17 52.07) (end 91.44 50.8) (width 0.25) (layer "F.Cu") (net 8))
 (segment (start 90.17 48.26) (end 77.47 48.26) (width 0.25) (layer "F.Cu") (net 8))
 (segment (start 88 52.07) (end 90.17 52.07) (width 0.25) (layer "F.Cu") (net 8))
 (segment (start 91.44 50.8) (end 91.44 49.53) (width 0.25) (layer "F.Cu") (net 8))
 (via (at 77.47 48.26) (size 0.8) (drill 0.4) (layers "F.Cu" "B.Cu") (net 8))
 (via (at 73.66 48.26) (size 0.8) (drill 0.4) (layers "F.Cu" "B.Cu") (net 8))
 (segment (start 73.66 48.26) (end 77.47 48.26) (width 0.25) (layer "B.Cu") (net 8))
 (segment (start 68.7316 48.49) (end 71.35 48.49) (width 0.25) (layer "F.Cu") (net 7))
 (segment (start 77.47 52.07) (end 82.18 52.07) (width 0.25) (layer "F.Cu") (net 7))
 (segment (start 71.35 48.49) (end 73.66 50.8) (width 0.25) (layer "F.Cu") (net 7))
 (via (at 77.47 52.07) (size 0.8) (drill 0.4) (layers "F.Cu" "B.Cu") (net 7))
 (via (at 73.66 50.8) (size 0.8) (drill 0.4) (layers "F.Cu" "B.Cu") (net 7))
 (segment (start 77.47 52.07) (end 74.93 52.07) (width 0.25) (layer "B.Cu") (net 7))
 (segment (start 73.66 50.8) (end 74.93 52.07) (width 0.25) (layer "B.Cu") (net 7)))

